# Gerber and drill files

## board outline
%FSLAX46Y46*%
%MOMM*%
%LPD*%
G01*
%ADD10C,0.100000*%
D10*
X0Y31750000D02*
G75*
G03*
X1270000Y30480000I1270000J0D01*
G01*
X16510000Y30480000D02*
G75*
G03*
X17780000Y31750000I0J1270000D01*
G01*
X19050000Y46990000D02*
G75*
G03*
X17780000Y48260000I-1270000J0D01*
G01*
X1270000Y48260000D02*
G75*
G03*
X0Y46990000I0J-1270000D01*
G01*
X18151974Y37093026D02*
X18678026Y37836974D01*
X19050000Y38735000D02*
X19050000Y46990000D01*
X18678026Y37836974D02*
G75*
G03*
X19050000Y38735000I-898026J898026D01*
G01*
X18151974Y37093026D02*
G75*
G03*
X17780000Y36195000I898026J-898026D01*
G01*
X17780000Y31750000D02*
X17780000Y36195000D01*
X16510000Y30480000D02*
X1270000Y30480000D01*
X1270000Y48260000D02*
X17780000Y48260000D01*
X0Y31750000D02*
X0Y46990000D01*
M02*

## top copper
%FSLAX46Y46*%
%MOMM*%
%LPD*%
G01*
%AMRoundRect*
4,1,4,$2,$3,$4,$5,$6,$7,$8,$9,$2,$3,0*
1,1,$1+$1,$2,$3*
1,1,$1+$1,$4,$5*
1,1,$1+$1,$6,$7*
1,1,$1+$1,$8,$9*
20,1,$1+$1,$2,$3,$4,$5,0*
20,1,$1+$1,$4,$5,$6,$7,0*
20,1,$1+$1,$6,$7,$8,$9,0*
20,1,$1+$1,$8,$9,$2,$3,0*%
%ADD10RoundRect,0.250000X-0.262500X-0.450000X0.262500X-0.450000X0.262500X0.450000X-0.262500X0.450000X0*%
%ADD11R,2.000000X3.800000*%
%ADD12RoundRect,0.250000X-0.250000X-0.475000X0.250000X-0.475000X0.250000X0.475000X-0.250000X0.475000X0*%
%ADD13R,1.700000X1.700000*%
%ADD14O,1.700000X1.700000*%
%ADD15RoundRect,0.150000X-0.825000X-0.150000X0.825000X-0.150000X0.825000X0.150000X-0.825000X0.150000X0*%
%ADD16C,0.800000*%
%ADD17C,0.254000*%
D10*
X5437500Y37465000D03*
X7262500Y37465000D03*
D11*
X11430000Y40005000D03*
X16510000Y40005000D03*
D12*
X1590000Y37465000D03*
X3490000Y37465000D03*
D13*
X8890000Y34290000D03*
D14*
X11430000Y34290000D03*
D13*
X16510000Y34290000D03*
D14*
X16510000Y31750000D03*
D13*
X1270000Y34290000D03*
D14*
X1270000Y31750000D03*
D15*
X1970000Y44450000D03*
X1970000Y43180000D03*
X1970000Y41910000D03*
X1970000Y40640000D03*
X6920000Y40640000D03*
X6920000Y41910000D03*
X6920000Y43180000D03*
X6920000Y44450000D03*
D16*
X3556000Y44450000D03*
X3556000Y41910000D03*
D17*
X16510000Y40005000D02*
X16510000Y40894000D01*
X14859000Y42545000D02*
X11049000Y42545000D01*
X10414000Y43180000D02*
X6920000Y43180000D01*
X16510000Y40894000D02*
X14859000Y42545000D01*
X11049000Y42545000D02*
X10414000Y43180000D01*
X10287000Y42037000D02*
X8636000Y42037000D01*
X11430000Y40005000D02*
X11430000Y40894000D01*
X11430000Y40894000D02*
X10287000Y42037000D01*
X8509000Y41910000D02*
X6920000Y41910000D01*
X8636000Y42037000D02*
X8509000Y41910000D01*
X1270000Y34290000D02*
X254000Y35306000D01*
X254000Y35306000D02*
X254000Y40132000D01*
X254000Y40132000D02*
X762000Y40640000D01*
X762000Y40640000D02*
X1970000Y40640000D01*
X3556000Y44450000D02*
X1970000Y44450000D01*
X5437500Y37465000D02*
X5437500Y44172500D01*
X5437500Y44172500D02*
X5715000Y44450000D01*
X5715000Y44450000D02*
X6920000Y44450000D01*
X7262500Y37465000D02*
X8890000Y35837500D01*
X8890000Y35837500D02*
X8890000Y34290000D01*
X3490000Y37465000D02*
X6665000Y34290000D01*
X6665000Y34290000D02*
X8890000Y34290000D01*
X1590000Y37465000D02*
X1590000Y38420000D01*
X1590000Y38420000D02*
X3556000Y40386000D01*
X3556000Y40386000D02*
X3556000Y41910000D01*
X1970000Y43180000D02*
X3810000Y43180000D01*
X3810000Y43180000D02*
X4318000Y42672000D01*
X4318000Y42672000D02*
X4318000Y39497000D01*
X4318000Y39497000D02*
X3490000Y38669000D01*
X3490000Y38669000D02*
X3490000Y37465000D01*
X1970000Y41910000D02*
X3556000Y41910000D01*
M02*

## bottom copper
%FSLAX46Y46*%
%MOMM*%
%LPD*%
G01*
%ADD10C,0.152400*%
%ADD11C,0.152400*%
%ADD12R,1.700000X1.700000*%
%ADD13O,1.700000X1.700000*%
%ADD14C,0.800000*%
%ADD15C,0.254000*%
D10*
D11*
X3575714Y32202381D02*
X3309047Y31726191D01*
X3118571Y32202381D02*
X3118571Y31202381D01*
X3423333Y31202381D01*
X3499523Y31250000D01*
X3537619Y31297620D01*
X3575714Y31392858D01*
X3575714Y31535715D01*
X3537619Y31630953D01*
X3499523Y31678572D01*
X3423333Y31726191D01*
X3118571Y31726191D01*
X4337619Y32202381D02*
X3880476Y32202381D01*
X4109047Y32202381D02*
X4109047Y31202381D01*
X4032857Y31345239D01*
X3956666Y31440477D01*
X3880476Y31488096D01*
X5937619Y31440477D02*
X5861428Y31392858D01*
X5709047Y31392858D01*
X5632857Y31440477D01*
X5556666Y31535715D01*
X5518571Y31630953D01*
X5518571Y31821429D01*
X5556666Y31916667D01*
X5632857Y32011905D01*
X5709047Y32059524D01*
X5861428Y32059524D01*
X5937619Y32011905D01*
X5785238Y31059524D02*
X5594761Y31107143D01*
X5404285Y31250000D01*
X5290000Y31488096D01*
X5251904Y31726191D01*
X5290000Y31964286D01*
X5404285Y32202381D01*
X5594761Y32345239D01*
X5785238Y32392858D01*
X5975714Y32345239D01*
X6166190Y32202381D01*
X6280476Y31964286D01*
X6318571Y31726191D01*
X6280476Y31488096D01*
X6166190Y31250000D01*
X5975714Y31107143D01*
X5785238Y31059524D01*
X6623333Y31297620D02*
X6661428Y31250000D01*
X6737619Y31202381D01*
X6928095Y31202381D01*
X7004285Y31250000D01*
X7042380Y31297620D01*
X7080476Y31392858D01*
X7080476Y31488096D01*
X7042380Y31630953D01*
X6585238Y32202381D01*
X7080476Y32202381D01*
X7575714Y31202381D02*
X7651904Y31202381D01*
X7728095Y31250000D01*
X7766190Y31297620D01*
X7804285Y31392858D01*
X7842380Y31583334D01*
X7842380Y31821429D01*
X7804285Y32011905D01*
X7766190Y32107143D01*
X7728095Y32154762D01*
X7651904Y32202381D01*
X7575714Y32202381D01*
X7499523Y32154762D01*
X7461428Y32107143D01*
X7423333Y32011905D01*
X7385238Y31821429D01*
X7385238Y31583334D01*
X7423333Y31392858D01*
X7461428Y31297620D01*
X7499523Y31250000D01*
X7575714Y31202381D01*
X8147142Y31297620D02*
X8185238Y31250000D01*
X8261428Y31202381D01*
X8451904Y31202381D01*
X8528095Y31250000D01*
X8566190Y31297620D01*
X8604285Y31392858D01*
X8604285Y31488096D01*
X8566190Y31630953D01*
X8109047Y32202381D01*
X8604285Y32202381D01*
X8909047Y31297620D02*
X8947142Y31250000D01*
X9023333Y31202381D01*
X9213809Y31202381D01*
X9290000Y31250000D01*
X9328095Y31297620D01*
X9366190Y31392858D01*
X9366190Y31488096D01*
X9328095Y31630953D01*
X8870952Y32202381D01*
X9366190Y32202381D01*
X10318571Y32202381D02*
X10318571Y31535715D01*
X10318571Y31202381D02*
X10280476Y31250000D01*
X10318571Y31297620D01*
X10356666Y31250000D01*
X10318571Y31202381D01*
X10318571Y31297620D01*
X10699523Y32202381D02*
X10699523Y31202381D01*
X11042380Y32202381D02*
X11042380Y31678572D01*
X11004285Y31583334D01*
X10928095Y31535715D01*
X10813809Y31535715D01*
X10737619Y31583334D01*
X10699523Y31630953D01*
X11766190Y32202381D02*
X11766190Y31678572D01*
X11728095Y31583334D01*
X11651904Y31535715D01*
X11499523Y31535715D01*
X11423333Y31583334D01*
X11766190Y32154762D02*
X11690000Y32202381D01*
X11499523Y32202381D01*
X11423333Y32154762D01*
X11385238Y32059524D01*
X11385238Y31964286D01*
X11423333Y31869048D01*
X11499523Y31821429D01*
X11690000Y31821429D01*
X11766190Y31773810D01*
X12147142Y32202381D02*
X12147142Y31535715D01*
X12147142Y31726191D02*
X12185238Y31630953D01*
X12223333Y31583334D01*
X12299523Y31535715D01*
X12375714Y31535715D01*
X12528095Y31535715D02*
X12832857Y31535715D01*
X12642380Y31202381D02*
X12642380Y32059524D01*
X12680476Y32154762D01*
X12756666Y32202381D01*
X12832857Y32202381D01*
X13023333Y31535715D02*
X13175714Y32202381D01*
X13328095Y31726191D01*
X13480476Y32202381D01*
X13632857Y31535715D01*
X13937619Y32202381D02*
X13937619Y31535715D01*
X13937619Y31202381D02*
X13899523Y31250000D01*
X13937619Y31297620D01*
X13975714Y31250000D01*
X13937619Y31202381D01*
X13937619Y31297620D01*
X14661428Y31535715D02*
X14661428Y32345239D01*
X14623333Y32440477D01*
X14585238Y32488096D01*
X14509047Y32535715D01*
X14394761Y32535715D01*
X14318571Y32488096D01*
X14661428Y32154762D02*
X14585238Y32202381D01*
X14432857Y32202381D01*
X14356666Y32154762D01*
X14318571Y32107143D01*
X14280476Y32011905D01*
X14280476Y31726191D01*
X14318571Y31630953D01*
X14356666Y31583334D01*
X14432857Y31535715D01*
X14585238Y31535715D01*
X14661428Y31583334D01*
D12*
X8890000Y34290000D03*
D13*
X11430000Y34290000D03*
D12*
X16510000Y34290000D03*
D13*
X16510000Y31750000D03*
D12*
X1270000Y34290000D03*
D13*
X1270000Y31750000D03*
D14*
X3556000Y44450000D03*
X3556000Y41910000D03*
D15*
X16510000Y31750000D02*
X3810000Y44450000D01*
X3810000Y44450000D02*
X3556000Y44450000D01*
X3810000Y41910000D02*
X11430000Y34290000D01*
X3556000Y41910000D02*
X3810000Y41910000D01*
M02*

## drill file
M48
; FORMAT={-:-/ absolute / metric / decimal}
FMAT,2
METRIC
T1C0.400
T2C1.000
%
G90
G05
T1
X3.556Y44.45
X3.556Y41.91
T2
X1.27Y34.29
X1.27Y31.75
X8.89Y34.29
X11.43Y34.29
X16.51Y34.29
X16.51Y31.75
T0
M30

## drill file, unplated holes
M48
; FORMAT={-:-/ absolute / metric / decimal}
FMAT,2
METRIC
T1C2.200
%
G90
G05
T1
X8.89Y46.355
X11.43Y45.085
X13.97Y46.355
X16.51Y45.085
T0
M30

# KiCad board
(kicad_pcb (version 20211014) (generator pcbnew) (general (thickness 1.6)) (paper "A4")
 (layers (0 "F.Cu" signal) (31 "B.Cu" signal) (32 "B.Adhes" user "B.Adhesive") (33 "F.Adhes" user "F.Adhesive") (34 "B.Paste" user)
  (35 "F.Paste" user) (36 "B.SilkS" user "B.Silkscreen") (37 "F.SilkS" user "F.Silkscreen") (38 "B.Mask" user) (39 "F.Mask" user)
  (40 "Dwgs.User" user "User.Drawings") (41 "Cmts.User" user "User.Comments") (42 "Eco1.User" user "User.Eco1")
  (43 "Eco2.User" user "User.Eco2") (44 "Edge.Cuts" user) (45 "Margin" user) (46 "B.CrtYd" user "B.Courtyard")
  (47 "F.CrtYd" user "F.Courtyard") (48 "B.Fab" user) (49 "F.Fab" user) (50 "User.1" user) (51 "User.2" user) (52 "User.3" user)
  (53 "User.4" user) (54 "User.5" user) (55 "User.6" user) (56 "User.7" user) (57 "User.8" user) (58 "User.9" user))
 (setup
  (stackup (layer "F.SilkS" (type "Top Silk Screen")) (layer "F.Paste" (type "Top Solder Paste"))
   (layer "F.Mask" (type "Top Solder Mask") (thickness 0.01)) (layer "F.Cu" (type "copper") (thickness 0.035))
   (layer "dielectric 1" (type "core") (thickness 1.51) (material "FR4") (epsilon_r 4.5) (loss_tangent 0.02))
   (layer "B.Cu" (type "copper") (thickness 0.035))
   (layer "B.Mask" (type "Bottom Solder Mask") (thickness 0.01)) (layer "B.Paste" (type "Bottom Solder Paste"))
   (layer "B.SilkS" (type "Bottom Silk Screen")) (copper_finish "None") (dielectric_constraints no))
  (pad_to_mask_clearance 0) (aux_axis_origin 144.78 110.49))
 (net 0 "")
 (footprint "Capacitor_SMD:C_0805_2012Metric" (layer "F.Cu") (at 147.32 73.025)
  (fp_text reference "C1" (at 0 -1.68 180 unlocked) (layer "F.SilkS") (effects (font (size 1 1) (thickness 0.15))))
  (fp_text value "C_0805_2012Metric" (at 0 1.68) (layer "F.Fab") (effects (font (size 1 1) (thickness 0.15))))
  (pad "1" smd roundrect (at -0.95 0) (size 1 1.45) (layers "F.Cu" "F.Paste" "F.Mask") (roundrect_rratio 0.25))
  (pad "2" smd roundrect (at 0.95 0) (size 1 1.45) (layers "F.Cu" "F.Paste" "F.Mask") (roundrect_rratio 0.25)))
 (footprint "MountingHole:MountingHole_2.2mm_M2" (layer "F.Cu") (at 158.75 64.135)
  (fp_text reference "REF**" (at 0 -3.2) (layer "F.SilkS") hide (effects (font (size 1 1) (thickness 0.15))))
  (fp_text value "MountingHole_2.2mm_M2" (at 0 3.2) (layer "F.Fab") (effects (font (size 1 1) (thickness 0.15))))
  (pad "" np_thru_hole circle (at 0 0) (size 2.2 2.2) (drill 2.2) (layers *.Cu *.Mask)))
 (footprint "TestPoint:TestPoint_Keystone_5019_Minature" (layer "F.Cu") (at 161.29 70.485 90)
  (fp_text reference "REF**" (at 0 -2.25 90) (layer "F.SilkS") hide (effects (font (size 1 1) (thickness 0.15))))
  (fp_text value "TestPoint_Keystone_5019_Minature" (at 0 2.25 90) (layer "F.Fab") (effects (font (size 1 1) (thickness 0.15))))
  (pad "1" smd rect (at 0 0 90) (size 3.8 2) (layers "F.Cu" "F.Paste" "F.Mask")))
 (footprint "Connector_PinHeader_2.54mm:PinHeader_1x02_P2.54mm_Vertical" (layer "F.Cu") (at 161.29 76.2)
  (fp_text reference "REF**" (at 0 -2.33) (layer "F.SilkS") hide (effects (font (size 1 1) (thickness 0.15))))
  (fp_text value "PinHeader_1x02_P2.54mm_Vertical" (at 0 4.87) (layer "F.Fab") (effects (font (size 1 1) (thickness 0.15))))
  (pad "1" thru_hole rect (at 0 0) (size 1.7 1.7) (drill 1) (layers *.Cu *.Mask))
  (pad "2" thru_hole oval (at 0 2.54) (size 1.7 1.7) (drill 1) (layers *.Cu *.Mask)))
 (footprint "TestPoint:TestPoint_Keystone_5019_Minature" (layer "F.Cu") (at 156.21 70.485 90)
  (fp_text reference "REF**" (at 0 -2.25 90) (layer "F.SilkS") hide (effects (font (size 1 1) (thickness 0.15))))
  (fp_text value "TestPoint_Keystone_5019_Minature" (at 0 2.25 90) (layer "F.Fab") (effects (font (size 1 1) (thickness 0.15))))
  (pad "1" smd rect (at 0 0 90) (size 3.8 2) (layers "F.Cu" "F.Paste" "F.Mask")))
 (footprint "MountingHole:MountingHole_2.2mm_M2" (layer "F.Cu") (at 153.67 64.135)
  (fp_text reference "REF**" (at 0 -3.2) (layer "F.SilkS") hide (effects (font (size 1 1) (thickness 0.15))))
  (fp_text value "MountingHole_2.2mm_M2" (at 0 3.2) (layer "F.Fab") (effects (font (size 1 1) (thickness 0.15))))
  (pad "" np_thru_hole circle (at 0 0) (size 2.2 2.2) (drill 2.2) (layers *.Cu *.Mask)))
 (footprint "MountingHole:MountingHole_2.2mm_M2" (layer "F.Cu") (at 161.29 65.405)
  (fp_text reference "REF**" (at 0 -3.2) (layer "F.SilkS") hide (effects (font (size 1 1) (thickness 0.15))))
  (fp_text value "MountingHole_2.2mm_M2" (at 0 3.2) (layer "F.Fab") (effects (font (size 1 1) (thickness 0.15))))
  (pad "" np_thru_hole circle (at 0 0) (size 2.2 2.2) (drill 2.2) (layers *.Cu *.Mask)))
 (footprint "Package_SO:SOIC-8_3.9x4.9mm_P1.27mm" (layer "F.Cu") (at 149.225 67.945)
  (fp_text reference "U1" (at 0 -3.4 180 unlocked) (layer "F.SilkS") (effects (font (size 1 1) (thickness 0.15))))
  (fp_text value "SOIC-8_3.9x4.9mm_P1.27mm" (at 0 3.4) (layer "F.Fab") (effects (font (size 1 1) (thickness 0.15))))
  (pad "1" smd roundrect (at -2.475 -1.905) (size 1.95 0.6) (layers "F.Cu" "F.Paste" "F.Mask") (roundrect_rratio 0.25))
  (pad "2" smd roundrect (at -2.475 -0.635) (size 1.95 0.6) (layers "F.Cu" "F.Paste" "F.Mask") (roundrect_rratio 0.25))
  (pad "3" smd roundrect (at -2.475 0.635) (size 1.95 0.6) (layers "F.Cu" "F.Paste" "F.Mask") (roundrect_rratio 0.25))
  (pad "4" smd roundrect (at -2.475 1.905) (size 1.95 0.6) (layers "F.Cu" "F.Paste" "F.Mask") (roundrect_rratio 0.25))
  (pad "5" smd roundrect (at 2.475 1.905) (size 1.95 0.6) (layers "F.Cu" "F.Paste" "F.Mask") (roundrect_rratio 0.25))
  (pad "6" smd roundrect (at 2.475 0.635) (size 1.95 0.6) (layers "F.Cu" "F.Paste" "F.Mask") (roundrect_rratio 0.25))
  (pad "7" smd roundrect (at 2.475 -0.635) (size 1.95 0.6) (layers "F.Cu" "F.Paste" "F.Mask") (roundrect_rratio 0.25))
  (pad "8" smd roundrect (at 2.475 -1.905) (size 1.95 0.6) (layers "F.Cu" "F.Paste" "F.Mask") (roundrect_rratio 0.25)))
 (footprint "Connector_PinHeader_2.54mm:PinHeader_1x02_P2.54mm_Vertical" (layer "F.Cu") (at 153.67 76.2 90)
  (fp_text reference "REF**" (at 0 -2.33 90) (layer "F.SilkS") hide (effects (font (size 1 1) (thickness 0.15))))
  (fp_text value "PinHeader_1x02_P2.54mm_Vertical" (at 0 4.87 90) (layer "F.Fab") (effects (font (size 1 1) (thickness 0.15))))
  (pad "1" thru_hole rect (at 0 0 90) (size 1.7 1.7) (drill 1) (layers *.Cu *.Mask))
  (pad "2" thru_hole oval (at 0 2.54 90) (size 1.7 1.7) (drill 1) (layers *.Cu *.Mask)))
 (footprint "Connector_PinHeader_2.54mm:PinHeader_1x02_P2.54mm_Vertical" (layer "F.Cu") (at 146.05 76.2)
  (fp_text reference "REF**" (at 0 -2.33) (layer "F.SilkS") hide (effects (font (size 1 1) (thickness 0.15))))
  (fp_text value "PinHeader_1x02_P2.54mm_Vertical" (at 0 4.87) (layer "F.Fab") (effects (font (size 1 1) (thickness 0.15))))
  (pad "1" thru_hole rect (at 0 0) (size 1.7 1.7) (drill 1) (layers *.Cu *.Mask))
  (pad "2" thru_hole oval (at 0 2.54) (size 1.7 1.7) (drill 1) (layers *.Cu *.Mask)))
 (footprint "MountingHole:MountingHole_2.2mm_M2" (layer "F.Cu") (at 156.21 65.405)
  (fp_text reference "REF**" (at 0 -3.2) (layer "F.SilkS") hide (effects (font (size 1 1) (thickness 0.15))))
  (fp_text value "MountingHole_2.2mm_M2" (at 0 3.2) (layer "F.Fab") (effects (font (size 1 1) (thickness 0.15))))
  (pad "" np_thru_hole circle (at 0 0) (size 2.2 2.2) (drill 2.2) (layers *.Cu *.Mask)))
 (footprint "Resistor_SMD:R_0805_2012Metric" (layer "F.Cu") (at 151.13 73.025)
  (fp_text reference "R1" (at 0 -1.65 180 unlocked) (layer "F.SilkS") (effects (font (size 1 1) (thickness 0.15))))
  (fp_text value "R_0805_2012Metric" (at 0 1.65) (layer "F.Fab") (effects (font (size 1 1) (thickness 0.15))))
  (pad "1" smd roundrect (at -0.9125 0) (size 1.025 1.4) (layers "F.Cu" "F.Paste" "F.Mask") (roundrect_rratio 0.243902439))
  (pad "2" smd roundrect (at 0.9125 0) (size 1.025 1.4) (layers "F.Cu" "F.Paste" "F.Mask") (roundrect_rratio 0.243902439)))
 (gr_line (start 162.56 78.74) (end 162.56 74.295) (layer "Edge.Cuts") (width 0.1))
 (gr_arc (start 162.56 74.295) (mid 162.656673 73.808992) (end 162.931974 73.396974) (layer "Edge.Cuts") (width 0.1))
 (gr_line (start 162.931974 73.396974) (end 163.458026 72.653026) (layer "Edge.Cuts") (width 0.1))
 (gr_line (start 163.83 71.755) (end 163.83 63.5) (layer "Edge.Cuts") (width 0.1))
 (gr_arc (start 162.56 78.74) (mid 162.188026 79.638026) (end 161.29 80.01) (layer "Edge.Cuts") (width 0.1))
 (gr_arc (start 146.05 80.01) (mid 145.151974 79.638026) (end 144.78 78.74) (layer "Edge.Cuts") (width 0.1))
 (gr_arc (start 144.78 63.5) (mid 145.151974 62.601974) (end 146.05 62.23) (layer "Edge.Cuts") (width 0.1))
 (gr_line (start 144.78 78.74) (end 144.78 63.5) (layer "Edge.Cuts") (width 0.1))
 (gr_arc (start 162.56 62.23) (mid 163.458026 62.601974) (end 163.83 63.5) (layer "Edge.Cuts") (width 0.1))
 (gr_line (start 161.29 80.01) (end 146.05 80.01) (layer "Edge.Cuts") (width 0.1))
 (gr_line (start 146.05 62.23) (end 162.56 62.23) (layer "Edge.Cuts") (width 0.1))
 (gr_arc (start 163.83 71.755) (mid 163.733327 72.241008) (end 163.458026 72.653026) (layer "Edge.Cuts") (width 0.1))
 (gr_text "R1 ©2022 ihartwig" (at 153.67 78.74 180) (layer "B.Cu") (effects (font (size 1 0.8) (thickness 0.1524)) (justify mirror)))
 (segment (start 156.21 69.596) (end 155.067 68.453) (width 0.254) (layer "F.Cu") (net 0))
 (segment (start 155.194 67.31) (end 151.7 67.31) (width 0.254) (layer "F.Cu") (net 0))
 (segment (start 145.034 70.358) (end 145.542 69.85) (width 0.254) (layer "F.Cu") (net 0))
 (segment (start 151.445 76.2) (end 153.67 76.2) (width 0.254) (layer "F.Cu") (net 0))
 (segment (start 150.495 66.04) (end 151.7 66.04) (width 0.254) (layer "F.Cu") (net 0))
 (segment (start 146.37 72.07) (end 148.336 70.104) (width 0.254) (layer "F.Cu") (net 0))
 (segment (start 148.336 66.04) (end 146.75 66.04) (width 0.254) (layer "F.Cu") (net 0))
 (segment (start 145.542 69.85) (end 146.75 69.85) (width 0.254) (layer "F.Cu") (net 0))
 (segment (start 155.829 67.945) (end 155.194 67.31) (width 0.254) (layer "F.Cu") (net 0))
 (segment (start 153.416 68.453) (end 153.289 68.58) (width 0.254) (layer "F.Cu") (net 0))
 (segment (start 145.034 75.184) (end 145.034 70.358) (width 0.254) (layer "F.Cu") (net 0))
 (segment (start 155.067 68.453) (end 153.416 68.453) (width 0.254) (layer "F.Cu") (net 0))
 (segment (start 150.2175 73.025) (end 150.2175 66.3175) (width 0.254) (layer "F.Cu") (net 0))
 (segment (start 156.21 70.485) (end 156.21 69.596) (width 0.254) (layer "F.Cu") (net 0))
 (segment (start 146.75 67.31) (end 148.59 67.31) (width 0.254) (layer "F.Cu") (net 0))
 (segment (start 159.639 67.945) (end 155.829 67.945) (width 0.254) (layer "F.Cu") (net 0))
 (segment (start 161.29 70.485) (end 161.29 69.596) (width 0.254) (layer "F.Cu") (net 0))
 (segment (start 146.37 73.025) (end 146.37 72.07) (width 0.254) (layer "F.Cu") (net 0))
 (segment (start 148.27 73.025) (end 151.445 76.2) (width 0.254) (layer "F.Cu") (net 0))
 (segment (start 161.29 69.596) (end 159.639 67.945) (width 0.254) (layer "F.Cu") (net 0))
 (segment (start 152.0425 73.025) (end 153.67 74.6525) (width 0.254) (layer "F.Cu") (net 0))
 (segment (start 153.289 68.58) (end 151.7 68.58) (width 0.254) (layer "F.Cu") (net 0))
 (segment (start 146.05 76.2) (end 145.034 75.184) (width 0.254) (layer "F.Cu") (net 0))
 (segment (start 148.336 70.104) (end 148.336 68.58) (width 0.254) (layer "F.Cu") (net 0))
 (segment (start 149.098 70.993) (end 148.27 71.821) (width 0.254) (layer "F.Cu") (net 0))
 (segment (start 150.2175 66.3175) (end 150.495 66.04) (width 0.254) (layer "F.Cu") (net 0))
 (segment (start 148.27 71.821) (end 148.27 73.025) (width 0.254) (layer "F.Cu") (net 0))
 (segment (start 153.67 74.6525) (end 153.67 76.2) (width 0.254) (layer "F.Cu") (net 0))
 (segment (start 148.59 67.31) (end 149.098 67.818) (width 0.254) (layer "F.Cu") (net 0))
 (segment (start 149.098 67.818) (end 149.098 70.993) (width 0.254) (layer "F.Cu") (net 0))
 (segment (start 146.75 68.58) (end 148.336 68.58) (width 0.254) (layer "F.Cu") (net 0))
 (via (at 148.336 66.04) (size 0.8) (drill 0.4) (layers "F.Cu" "B.Cu") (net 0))
 (via (at 148.336 68.58) (size 0.8) (drill 0.4) (layers "F.Cu" "B.Cu") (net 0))
 (segment (start 161.29 78.74) (end 148.59 66.04) (width 0.254) (layer "B.Cu") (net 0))
 (segment (start 148.59 68.58) (end 156.21 76.2) (width 0.254) (layer "B.Cu") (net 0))
 (segment (start 148.59 66.04) (end 148.336 66.04) (width 0.254) (layer "B.Cu") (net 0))
 (segment (start 148.336 68.58) (end 148.59 68.58) (width 0.254) (layer "B.Cu") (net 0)))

